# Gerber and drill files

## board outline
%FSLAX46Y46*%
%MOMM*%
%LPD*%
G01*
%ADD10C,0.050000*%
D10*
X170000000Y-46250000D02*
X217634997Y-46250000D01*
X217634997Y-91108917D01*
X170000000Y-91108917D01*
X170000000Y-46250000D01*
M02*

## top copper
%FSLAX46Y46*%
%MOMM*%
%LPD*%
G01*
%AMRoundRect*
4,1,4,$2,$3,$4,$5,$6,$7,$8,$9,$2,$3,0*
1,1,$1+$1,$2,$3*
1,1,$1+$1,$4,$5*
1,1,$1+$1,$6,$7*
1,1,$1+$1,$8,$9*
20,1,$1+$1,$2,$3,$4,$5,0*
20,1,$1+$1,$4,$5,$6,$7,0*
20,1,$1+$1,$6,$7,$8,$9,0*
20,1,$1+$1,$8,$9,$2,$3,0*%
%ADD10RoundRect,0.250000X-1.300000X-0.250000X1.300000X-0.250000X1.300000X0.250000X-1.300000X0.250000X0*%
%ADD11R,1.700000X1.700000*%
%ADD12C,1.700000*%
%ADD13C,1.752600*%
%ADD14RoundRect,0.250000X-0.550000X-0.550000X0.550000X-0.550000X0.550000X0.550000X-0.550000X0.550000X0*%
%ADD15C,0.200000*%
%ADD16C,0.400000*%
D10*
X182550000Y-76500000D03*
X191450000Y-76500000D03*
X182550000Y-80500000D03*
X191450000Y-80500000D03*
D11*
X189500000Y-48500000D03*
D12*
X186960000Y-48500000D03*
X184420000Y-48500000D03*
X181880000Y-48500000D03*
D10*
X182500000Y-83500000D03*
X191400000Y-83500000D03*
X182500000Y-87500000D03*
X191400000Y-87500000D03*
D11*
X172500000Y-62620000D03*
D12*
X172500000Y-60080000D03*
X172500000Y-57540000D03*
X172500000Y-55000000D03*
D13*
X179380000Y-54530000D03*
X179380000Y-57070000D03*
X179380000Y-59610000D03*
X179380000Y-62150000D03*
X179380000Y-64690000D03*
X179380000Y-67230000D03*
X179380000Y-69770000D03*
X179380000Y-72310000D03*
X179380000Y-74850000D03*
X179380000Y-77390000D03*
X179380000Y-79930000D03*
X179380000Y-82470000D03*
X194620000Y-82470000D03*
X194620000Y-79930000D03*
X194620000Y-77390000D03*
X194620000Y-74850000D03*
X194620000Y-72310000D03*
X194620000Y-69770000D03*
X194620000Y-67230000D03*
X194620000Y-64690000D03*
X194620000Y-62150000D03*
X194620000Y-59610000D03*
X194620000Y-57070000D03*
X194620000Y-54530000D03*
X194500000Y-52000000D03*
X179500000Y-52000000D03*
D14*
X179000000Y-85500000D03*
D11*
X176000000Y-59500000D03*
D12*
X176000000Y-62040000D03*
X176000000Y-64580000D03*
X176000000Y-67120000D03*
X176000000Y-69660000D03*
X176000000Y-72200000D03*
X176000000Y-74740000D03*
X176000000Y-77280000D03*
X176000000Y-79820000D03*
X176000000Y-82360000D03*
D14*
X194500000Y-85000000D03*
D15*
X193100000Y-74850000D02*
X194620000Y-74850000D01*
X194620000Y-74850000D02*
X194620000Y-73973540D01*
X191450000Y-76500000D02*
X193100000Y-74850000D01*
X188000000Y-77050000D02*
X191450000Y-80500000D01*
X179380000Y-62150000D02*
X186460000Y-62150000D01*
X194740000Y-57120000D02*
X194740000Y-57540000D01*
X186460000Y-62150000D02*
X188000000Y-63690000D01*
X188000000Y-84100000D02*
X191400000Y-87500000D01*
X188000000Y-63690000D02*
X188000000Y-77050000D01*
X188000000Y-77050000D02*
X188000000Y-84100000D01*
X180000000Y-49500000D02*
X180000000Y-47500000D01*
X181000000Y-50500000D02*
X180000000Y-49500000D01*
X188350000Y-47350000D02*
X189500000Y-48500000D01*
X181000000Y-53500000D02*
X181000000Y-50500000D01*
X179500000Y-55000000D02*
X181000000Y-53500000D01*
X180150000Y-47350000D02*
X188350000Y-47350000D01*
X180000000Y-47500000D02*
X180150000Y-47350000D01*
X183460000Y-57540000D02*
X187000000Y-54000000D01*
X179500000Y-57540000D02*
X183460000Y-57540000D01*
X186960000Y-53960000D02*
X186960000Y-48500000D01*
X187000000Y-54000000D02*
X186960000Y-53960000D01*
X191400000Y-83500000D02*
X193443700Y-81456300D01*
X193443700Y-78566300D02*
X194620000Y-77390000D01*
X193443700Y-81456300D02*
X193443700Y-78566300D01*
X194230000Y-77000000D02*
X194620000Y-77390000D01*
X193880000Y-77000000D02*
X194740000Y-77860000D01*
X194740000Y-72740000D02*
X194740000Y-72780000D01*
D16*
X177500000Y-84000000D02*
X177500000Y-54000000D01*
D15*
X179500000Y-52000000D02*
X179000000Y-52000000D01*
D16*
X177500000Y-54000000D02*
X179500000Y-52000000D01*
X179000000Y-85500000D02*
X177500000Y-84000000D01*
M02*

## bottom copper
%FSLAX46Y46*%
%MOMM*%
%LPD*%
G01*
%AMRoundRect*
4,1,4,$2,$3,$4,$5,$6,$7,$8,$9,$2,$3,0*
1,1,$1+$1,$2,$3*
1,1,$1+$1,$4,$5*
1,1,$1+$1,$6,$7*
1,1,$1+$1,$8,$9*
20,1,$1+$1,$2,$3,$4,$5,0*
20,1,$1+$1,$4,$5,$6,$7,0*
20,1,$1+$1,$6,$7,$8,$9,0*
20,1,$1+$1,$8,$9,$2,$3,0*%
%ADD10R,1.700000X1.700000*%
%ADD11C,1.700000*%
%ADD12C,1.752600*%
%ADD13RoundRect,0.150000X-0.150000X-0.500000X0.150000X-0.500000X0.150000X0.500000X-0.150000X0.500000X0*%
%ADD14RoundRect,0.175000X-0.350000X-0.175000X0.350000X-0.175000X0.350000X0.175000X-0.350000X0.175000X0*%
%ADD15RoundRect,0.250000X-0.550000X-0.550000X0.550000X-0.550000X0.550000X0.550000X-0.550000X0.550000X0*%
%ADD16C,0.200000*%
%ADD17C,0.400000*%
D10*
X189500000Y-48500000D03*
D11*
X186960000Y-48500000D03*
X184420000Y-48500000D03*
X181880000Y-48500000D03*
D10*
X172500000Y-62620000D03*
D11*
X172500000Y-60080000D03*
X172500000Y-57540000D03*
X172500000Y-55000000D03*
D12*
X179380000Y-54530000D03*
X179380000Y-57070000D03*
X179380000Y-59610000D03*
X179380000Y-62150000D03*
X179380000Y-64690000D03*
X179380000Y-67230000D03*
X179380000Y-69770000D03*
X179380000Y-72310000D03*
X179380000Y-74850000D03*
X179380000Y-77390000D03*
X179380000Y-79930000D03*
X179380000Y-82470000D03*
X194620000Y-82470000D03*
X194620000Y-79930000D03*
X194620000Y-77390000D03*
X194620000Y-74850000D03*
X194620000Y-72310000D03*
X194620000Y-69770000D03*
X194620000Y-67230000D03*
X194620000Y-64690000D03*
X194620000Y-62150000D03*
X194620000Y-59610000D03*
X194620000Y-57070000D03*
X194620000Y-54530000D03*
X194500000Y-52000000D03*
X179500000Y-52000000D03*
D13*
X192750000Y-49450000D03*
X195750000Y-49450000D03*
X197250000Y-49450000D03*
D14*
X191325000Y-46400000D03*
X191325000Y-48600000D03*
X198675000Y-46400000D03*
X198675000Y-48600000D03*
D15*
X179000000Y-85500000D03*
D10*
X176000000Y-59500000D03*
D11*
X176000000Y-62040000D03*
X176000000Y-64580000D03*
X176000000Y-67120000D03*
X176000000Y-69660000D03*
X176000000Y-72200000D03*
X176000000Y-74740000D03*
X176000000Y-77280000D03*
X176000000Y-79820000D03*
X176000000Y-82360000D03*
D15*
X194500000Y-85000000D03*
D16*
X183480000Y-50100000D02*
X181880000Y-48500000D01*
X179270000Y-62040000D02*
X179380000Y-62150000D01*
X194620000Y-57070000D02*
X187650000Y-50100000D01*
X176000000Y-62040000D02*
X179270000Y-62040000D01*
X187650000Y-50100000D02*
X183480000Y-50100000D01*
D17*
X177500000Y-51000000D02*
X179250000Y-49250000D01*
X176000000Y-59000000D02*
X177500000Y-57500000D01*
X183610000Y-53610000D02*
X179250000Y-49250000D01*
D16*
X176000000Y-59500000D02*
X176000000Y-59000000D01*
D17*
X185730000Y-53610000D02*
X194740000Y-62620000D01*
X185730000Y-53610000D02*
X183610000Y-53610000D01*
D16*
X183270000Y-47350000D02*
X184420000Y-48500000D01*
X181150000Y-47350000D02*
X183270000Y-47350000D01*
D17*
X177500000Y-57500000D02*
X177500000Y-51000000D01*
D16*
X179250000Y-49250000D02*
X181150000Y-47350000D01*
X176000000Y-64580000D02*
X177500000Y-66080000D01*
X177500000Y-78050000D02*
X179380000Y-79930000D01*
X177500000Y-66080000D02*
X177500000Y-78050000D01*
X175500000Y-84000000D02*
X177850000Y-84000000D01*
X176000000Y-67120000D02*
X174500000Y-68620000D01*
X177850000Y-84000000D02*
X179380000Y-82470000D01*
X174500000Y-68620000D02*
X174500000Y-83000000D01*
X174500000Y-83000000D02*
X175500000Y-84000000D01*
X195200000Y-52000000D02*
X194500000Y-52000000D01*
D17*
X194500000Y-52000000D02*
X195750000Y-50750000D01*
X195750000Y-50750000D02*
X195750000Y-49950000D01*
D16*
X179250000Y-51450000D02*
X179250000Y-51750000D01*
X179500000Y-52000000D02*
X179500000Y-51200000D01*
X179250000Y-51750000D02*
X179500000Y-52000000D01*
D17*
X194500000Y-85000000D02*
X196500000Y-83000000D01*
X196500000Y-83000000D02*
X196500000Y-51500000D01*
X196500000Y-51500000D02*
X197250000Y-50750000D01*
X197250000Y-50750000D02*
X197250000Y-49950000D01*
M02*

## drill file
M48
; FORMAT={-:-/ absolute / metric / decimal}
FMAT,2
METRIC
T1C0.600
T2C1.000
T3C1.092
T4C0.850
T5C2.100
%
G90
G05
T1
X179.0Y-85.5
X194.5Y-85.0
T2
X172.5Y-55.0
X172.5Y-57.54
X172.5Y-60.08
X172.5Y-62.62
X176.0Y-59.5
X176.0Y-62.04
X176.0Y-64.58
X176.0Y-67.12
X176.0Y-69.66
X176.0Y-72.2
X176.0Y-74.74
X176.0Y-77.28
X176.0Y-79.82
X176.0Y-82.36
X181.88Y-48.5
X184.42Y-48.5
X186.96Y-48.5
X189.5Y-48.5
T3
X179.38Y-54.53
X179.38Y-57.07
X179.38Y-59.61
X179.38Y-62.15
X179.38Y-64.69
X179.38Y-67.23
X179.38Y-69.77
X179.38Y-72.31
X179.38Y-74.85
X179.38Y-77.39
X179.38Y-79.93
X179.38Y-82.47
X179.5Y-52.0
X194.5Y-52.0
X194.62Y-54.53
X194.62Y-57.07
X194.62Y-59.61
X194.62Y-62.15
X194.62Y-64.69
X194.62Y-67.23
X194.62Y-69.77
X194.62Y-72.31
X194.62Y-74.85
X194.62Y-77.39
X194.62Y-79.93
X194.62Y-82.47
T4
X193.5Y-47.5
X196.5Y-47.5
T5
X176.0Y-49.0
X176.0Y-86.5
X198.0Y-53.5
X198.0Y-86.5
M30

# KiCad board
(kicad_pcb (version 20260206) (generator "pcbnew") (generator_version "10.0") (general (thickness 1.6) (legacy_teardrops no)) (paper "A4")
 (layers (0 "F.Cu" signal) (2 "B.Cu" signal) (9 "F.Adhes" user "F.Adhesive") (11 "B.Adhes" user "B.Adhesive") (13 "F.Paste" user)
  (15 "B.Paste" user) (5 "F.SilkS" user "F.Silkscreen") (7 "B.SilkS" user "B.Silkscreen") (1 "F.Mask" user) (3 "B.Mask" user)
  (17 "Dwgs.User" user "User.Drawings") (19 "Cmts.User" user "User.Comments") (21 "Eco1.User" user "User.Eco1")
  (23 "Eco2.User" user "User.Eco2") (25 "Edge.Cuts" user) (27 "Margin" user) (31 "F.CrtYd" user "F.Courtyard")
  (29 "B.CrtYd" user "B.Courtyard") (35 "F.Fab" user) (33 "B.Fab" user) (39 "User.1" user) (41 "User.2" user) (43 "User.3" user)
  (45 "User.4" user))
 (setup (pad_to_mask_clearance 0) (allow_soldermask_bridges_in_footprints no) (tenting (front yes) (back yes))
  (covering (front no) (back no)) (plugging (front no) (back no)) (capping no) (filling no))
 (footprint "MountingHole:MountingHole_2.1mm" (layer "F.Cu") (at 176 49)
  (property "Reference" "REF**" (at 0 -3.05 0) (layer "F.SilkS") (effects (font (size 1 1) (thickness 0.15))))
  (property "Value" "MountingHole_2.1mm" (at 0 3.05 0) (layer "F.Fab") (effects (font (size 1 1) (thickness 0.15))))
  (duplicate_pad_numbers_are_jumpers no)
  (pad "" np_thru_hole circle (at 0 0) (size 2.1 2.1) (drill 2.1) (layers "*.Cu" "*.Mask")))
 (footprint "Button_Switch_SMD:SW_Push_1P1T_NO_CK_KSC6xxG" (layer "F.Cu") (at 187 78.5)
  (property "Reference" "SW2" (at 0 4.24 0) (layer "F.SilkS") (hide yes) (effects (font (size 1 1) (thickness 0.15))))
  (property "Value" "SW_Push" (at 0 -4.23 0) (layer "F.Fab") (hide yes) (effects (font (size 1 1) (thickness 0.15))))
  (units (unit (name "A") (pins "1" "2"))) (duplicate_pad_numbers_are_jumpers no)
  (pad "1" smd roundrect (at -4.45 -2) (size 3.1 1) (layers "F.Cu" "F.Mask" "F.Paste") (roundrect_rratio 0.25) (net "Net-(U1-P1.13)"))
  (pad "1" smd roundrect (at 4.45 -2) (size 3.1 1) (layers "F.Cu" "F.Mask" "F.Paste") (roundrect_rratio 0.25) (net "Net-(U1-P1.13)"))
  (pad "2" smd roundrect (at -4.45 2) (size 3.1 1) (layers "F.Cu" "F.Mask" "F.Paste") (roundrect_rratio 0.25) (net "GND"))
  (pad "2" smd roundrect (at 4.45 2) (size 3.1 1) (layers "F.Cu" "F.Mask" "F.Paste") (roundrect_rratio 0.25) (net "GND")))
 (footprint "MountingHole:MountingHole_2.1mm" (layer "F.Cu") (at 198 86.5)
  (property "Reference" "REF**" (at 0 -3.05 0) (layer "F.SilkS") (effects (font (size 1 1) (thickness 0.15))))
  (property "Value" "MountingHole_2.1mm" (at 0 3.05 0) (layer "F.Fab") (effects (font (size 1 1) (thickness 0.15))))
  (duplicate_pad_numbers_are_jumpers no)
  (pad "" np_thru_hole circle (at 0 0) (size 2.1 2.1) (drill 2.1) (layers "*.Cu" "*.Mask")))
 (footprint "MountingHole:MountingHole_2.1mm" (layer "F.Cu") (at 176 86.5)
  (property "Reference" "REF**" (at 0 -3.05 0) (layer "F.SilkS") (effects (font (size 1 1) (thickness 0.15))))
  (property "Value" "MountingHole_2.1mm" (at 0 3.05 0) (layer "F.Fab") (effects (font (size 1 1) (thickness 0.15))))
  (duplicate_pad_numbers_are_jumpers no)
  (pad "" np_thru_hole circle (at 0 0) (size 2.1 2.1) (drill 2.1) (layers "*.Cu" "*.Mask")))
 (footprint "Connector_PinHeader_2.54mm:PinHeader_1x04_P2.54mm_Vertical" (layer "F.Cu") (at 189.5 48.5 -90)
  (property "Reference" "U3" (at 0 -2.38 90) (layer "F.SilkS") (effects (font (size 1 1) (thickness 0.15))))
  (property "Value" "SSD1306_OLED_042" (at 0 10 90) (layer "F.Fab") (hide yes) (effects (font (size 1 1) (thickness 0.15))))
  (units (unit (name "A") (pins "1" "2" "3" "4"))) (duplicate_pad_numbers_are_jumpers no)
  (pad "1" thru_hole rect (at 0 0 270) (size 1.7 1.7) (drill 1) (layers "*.Cu" "*.Mask") (remove_unused_layers no)
   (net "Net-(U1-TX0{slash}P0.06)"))
  (pad "2" thru_hole circle (at 0 2.54 270) (size 1.7 1.7) (drill 1) (layers "*.Cu" "*.Mask") (remove_unused_layers no)
   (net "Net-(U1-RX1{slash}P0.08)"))
  (pad "3" thru_hole circle (at 0 5.08 270) (size 1.7 1.7) (drill 1) (layers "*.Cu" "*.Mask") (remove_unused_layers no) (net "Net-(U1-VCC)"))
  (pad "4" thru_hole circle (at 0 7.62 270) (size 1.7 1.7) (drill 1) (layers "*.Cu" "*.Mask") (remove_unused_layers no) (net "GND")))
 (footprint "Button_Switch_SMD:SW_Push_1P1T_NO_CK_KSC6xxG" (layer "F.Cu") (at 186.95 85.5)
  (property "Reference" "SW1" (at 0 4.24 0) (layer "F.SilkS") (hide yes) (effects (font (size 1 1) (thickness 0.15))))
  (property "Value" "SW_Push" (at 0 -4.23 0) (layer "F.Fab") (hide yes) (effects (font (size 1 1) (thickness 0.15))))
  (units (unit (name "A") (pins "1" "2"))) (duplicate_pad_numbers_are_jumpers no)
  (pad "1" smd roundrect (at -4.45 -2) (size 3.1 1) (layers "F.Cu" "F.Mask" "F.Paste") (roundrect_rratio 0.25) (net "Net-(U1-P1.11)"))
  (pad "1" smd roundrect (at 4.45 -2) (size 3.1 1) (layers "F.Cu" "F.Mask" "F.Paste") (roundrect_rratio 0.25) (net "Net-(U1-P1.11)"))
  (pad "2" smd roundrect (at -4.45 2) (size 3.1 1) (layers "F.Cu" "F.Mask" "F.Paste") (roundrect_rratio 0.25) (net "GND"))
  (pad "2" smd roundrect (at 4.45 2) (size 3.1 1) (layers "F.Cu" "F.Mask" "F.Paste") (roundrect_rratio 0.25) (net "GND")))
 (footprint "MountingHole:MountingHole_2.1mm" (layer "F.Cu") (at 198 53.5)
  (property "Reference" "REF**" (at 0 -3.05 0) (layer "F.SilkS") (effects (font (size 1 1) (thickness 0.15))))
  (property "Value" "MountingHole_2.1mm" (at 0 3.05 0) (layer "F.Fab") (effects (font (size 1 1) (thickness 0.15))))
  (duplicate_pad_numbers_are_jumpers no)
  (pad "" np_thru_hole circle (at 0 0) (size 2.1 2.1) (drill 2.1) (layers "*.Cu" "*.Mask")))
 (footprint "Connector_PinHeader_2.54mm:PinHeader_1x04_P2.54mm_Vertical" (layer "F.Cu") (at 172.5 62.62 180)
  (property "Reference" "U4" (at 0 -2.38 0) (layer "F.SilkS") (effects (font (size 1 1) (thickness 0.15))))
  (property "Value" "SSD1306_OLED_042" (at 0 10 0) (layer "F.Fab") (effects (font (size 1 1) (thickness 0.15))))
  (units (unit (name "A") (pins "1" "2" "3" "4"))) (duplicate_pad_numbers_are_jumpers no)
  (pad "1" thru_hole rect (at 0 0 180) (size 1.7 1.7) (drill 1) (layers "*.Cu" "*.Mask") (remove_unused_layers no)
   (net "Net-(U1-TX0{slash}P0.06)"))
  (pad "2" thru_hole circle (at 0 2.54 180) (size 1.7 1.7) (drill 1) (layers "*.Cu" "*.Mask") (remove_unused_layers no)
   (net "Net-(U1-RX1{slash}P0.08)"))
  (pad "3" thru_hole circle (at 0 5.08 180) (size 1.7 1.7) (drill 1) (layers "*.Cu" "*.Mask") (remove_unused_layers no) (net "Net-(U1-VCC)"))
  (pad "4" thru_hole circle (at 0 7.62 180) (size 1.7 1.7) (drill 1) (layers "*.Cu" "*.Mask") (remove_unused_layers no) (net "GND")))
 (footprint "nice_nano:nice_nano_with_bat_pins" (layer "F.Cu") (at 187 68.5 -90)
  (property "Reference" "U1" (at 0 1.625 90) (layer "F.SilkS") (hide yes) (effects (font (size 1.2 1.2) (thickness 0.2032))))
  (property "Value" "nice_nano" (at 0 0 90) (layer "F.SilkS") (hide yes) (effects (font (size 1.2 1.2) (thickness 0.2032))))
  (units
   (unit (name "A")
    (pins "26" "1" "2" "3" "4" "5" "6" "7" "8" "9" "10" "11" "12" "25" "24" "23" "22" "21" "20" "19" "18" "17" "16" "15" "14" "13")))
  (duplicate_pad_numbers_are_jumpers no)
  (pad "1" thru_hole circle (at -13.97 7.62 270) (size 1.7526 1.7526) (drill 1.0922) (layers "*.Cu" "*.SilkS" "*.Mask")
   (remove_unused_layers no) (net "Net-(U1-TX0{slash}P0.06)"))
  (pad "2" thru_hole circle (at -11.43 7.62 270) (size 1.7526 1.7526) (drill 1.0922) (layers "*.Cu" "*.SilkS" "*.Mask")
   (remove_unused_layers no) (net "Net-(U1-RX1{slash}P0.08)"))
  (pad "3" thru_hole circle (at -8.89 7.62 270) (size 1.7526 1.7526) (drill 1.0922) (layers "*.Cu" "*.SilkS" "*.Mask")
   (remove_unused_layers no) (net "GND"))
  (pad "4" thru_hole circle (at -6.35 7.62 270) (size 1.7526 1.7526) (drill 1.0922) (layers "*.Cu" "*.SilkS" "*.Mask")
   (remove_unused_layers no) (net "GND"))
  (pad "5" thru_hole circle (at -3.81 7.62 270) (size 1.7526 1.7526) (drill 1.0922) (layers "*.Cu" "*.SilkS" "*.Mask")
   (remove_unused_layers no) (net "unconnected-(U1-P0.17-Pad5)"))
  (pad "6" thru_hole circle (at -1.27 7.62 270) (size 1.7526 1.7526) (drill 1.0922) (layers "*.Cu" "*.SilkS" "*.Mask")
   (remove_unused_layers no) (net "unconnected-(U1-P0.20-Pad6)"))
  (pad "7" thru_hole circle (at 1.27 7.62 270) (size 1.7526 1.7526) (drill 1.0922) (layers "*.Cu" "*.SilkS" "*.Mask")
   (remove_unused_layers no) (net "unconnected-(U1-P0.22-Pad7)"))
  (pad "8" thru_hole circle (at 3.81 7.62 270) (size 1.7526 1.7526) (drill 1.0922) (layers "*.Cu" "*.SilkS" "*.Mask")
   (remove_unused_layers no) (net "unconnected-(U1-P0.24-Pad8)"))
  (pad "9" thru_hole circle (at 6.35 7.62 270) (size 1.7526 1.7526) (drill 1.0922) (layers "*.Cu" "*.SilkS" "*.Mask")
   (remove_unused_layers no) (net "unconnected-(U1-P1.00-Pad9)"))
  (pad "10" thru_hole circle (at 8.89 7.62 270) (size 1.7526 1.7526) (drill 1.0922) (layers "*.Cu" "*.SilkS" "*.Mask")
   (remove_unused_layers no) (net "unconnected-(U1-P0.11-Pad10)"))
  (pad "11" thru_hole circle (at 11.43 7.62 270) (size 1.7526 1.7526) (drill 1.0922) (layers "*.Cu" "*.SilkS" "*.Mask")
   (remove_unused_layers no) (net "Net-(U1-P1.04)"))
  (pad "12" thru_hole circle (at 13.97 7.62 270) (size 1.7526 1.7526) (drill 1.0922) (layers "*.Cu" "*.SilkS" "*.Mask")
   (remove_unused_layers no) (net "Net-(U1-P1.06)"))
  (pad "13" thru_hole circle (at 13.97 -7.62 270) (size 1.7526 1.7526) (drill 1.0922) (layers "*.Cu" "*.SilkS" "*.Mask")
   (remove_unused_layers no) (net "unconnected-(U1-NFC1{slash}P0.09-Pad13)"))
  (pad "14" thru_hole circle (at 11.43 -7.62 270) (size 1.7526 1.7526) (drill 1.0922) (layers "*.Cu" "*.SilkS" "*.Mask")
   (remove_unused_layers no) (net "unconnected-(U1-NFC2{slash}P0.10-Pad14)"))
  (pad "15" thru_hole circle (at 8.89 -7.62 270) (size 1.7526 1.7526) (drill 1.0922) (layers "*.Cu" "*.SilkS" "*.Mask")
   (remove_unused_layers no) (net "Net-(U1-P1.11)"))
  (pad "16" thru_hole circle (at 6.35 -7.62 270) (size 1.7526 1.7526) (drill 1.0922) (layers "*.Cu" "*.SilkS" "*.Mask")
   (remove_unused_layers no) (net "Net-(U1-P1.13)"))
  (pad "17" thru_hole circle (at 3.81 -7.62 270) (size 1.7526 1.7526) (drill 1.0922) (layers "*.Cu" "*.SilkS" "*.Mask")
   (remove_unused_layers no) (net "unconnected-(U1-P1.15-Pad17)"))
  (pad "18" thru_hole circle (at 1.27 -7.62 270) (size 1.7526 1.7526) (drill 1.0922) (layers "*.Cu" "*.SilkS" "*.Mask")
   (remove_unused_layers no) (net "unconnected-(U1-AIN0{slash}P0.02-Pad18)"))
  (pad "19" thru_hole circle (at -1.27 -7.62 270) (size 1.7526 1.7526) (drill 1.0922) (layers "*.Cu" "*.SilkS" "*.Mask")
   (remove_unused_layers no) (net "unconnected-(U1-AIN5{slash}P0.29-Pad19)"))
  (pad "20" thru_hole circle (at -3.81 -7.62 270) (size 1.7526 1.7526) (drill 1.0922) (layers "*.Cu" "*.SilkS" "*.Mask")
   (remove_unused_layers no) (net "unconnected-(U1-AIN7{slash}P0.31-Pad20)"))
  (pad "21" thru_hole circle (at -6.35 -7.62 270) (size 1.7526 1.7526) (drill 1.0922) (layers "*.Cu" "*.SilkS" "*.Mask")
   (remove_unused_layers no) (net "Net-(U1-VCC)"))
  (pad "22" thru_hole circle (at -8.89 -7.62 270) (size 1.7526 1.7526) (drill 1.0922) (layers "*.Cu" "*.SilkS" "*.Mask")
   (remove_unused_layers no) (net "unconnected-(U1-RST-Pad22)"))
  (pad "23" thru_hole circle (at -11.43 -7.62 270) (size 1.7526 1.7526) (drill 1.0922) (layers "*.Cu" "*.SilkS" "*.Mask")
   (remove_unused_layers no) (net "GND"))
  (pad "24" thru_hole circle (at -13.97 -7.62 270) (size 1.7526 1.7526) (drill 1.0922) (layers "*.Cu" "*.SilkS" "*.Mask")
   (remove_unused_layers no) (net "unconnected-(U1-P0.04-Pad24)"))
  (pad "25" thru_hole circle (at -16.5 -7.5 270) (size 1.7526 1.7526) (drill 1.0922) (layers "*.Cu" "*.SilkS" "*.Mask")
   (remove_unused_layers no) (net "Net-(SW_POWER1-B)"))
  (pad "26" thru_hole circle (at -16.5 7.5 270) (size 1.7526 1.7526) (drill 1.0922) (layers "*.Cu" "*.SilkS" "*.Mask")
   (remove_unused_layers no) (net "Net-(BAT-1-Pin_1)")))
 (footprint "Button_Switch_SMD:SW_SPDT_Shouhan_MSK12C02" (layer "B.Cu") (at 195 47.5)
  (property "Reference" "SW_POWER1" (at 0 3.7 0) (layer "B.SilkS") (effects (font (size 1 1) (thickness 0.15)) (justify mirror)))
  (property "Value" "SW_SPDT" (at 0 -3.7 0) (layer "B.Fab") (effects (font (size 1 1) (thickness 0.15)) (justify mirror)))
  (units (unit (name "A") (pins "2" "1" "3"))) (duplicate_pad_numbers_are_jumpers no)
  (pad "" np_thru_hole circle (at -1.5 0) (size 0.85 0.85) (drill 0.85) (layers "*.Mask"))
  (pad "" np_thru_hole circle (at 1.5 0) (size 0.85 0.85) (drill 0.85) (layers "*.Mask"))
  (pad "1" smd roundrect (at -2.25 1.95) (size 0.6 1.3) (layers "B.Cu" "B.Mask" "B.Paste") (roundrect_rratio 0.25)
   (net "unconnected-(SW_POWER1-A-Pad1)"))
  (pad "2" smd roundrect (at 0.75 1.95) (size 0.6 1.3) (layers "B.Cu" "B.Mask" "B.Paste") (roundrect_rratio 0.25) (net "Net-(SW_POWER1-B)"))
  (pad "3" smd roundrect (at 2.25 1.95) (size 0.6 1.3) (layers "B.Cu" "B.Mask" "B.Paste") (roundrect_rratio 0.25) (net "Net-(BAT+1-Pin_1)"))
  (pad "SH" smd roundrect (at -3.675 -1.1) (size 1.05 0.7) (layers "B.Cu" "B.Mask" "B.Paste") (roundrect_rratio 0.25))
  (pad "SH" smd roundrect (at -3.675 1.1) (size 1.05 0.7) (layers "B.Cu" "B.Mask" "B.Paste") (roundrect_rratio 0.25))
  (pad "SH" smd roundrect (at 3.675 -1.1) (size 1.05 0.7) (layers "B.Cu" "B.Mask" "B.Paste") (roundrect_rratio 0.25))
  (pad "SH" smd roundrect (at 3.675 1.1) (size 1.05 0.7) (layers "B.Cu" "B.Mask" "B.Paste") (roundrect_rratio 0.25)))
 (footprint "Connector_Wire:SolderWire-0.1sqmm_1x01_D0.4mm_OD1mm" (layer "B.Cu") (at 179 85.5)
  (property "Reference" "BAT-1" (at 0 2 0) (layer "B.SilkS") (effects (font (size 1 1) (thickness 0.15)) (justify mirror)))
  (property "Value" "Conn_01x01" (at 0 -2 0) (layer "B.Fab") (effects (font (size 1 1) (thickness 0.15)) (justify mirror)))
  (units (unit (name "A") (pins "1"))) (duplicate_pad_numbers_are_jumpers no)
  (pad "1" thru_hole roundrect (at 0 0) (size 1.6 1.6) (drill 0.6) (layers "*.Cu" "*.Mask") (remove_unused_layers no)
   (roundrect_rratio 0.15625) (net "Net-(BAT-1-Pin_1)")))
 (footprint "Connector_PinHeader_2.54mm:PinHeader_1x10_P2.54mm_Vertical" (layer "B.Cu") (at 176 59.5 180)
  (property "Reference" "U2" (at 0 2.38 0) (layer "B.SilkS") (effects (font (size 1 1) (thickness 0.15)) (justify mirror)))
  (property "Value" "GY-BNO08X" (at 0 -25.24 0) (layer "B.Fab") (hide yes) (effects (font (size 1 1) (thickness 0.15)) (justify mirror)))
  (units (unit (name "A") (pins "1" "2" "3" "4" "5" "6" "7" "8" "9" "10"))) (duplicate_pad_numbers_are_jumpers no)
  (pad "1" thru_hole rect (at 0 0 180) (size 1.7 1.7) (drill 1) (layers "*.Cu" "*.Mask") (remove_unused_layers no) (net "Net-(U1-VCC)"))
  (pad "2" thru_hole circle (at 0 -2.54 180) (size 1.7 1.7) (drill 1) (layers "*.Cu" "*.Mask") (remove_unused_layers no) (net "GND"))
  (pad "3" thru_hole circle (at 0 -5.08 180) (size 1.7 1.7) (drill 1) (layers "*.Cu" "*.Mask") (remove_unused_layers no)
   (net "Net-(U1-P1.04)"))
  (pad "4" thru_hole circle (at 0 -7.62 180) (size 1.7 1.7) (drill 1) (layers "*.Cu" "*.Mask") (remove_unused_layers no)
   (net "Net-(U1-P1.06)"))
  (pad "5" thru_hole circle (at 0 -10.16 180) (size 1.7 1.7) (drill 1) (layers "*.Cu" "*.Mask") (remove_unused_layers no)
   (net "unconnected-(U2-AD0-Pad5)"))
  (pad "6" thru_hole circle (at 0 -12.7 180) (size 1.7 1.7) (drill 1) (layers "*.Cu" "*.Mask") (remove_unused_layers no)
   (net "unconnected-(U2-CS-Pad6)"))
  (pad "7" thru_hole circle (at 0 -15.24 180) (size 1.7 1.7) (drill 1) (layers "*.Cu" "*.Mask") (remove_unused_layers no)
   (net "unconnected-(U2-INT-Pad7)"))
  (pad "8" thru_hole circle (at 0 -17.78 180) (size 1.7 1.7) (drill 1) (layers "*.Cu" "*.Mask") (remove_unused_layers no)
   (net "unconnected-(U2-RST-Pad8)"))
  (pad "9" thru_hole circle (at 0 -20.32 180) (size 1.7 1.7) (drill 1) (layers "*.Cu" "*.Mask") (remove_unused_layers no)
   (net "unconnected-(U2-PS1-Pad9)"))
  (pad "10" thru_hole circle (at 0 -22.86 180) (size 1.7 1.7) (drill 1) (layers "*.Cu" "*.Mask") (remove_unused_layers no)
   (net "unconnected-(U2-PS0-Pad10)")))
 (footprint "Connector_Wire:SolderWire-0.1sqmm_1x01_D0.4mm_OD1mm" (layer "B.Cu") (at 194.5 85)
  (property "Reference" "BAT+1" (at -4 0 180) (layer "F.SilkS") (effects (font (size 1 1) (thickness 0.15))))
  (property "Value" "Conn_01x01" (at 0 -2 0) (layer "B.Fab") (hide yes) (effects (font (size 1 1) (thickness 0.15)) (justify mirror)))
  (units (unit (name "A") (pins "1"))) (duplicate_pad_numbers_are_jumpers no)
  (pad "1" thru_hole roundrect (at 0 0) (size 1.6 1.6) (drill 0.6) (layers "*.Cu" "*.Mask") (remove_unused_layers no)
   (roundrect_rratio 0.15625) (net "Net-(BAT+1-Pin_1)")))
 (gr_rect (start 170 46.25) (end 217.634997 91.108917) (stroke (width 0.05) (type default)) (fill no) (layer "Edge.Cuts"))
 (segment (start 193.1 74.85) (end 194.62 74.85) (width 0.2) (layer "F.Cu") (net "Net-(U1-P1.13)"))
 (segment (start 194.62 74.85) (end 194.62 73.97354) (width 0.2) (layer "F.Cu") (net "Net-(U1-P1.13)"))
 (segment (start 191.45 76.5) (end 193.1 74.85) (width 0.2) (layer "F.Cu") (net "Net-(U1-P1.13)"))
 (segment (start 188 77.05) (end 191.45 80.5) (width 0.2) (layer "F.Cu") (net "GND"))
 (segment (start 179.38 62.15) (end 186.46 62.15) (width 0.2) (layer "F.Cu") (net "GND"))
 (segment (start 194.74 57.12) (end 194.74 57.54) (width 0.2) (layer "F.Cu") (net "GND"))
 (segment (start 186.46 62.15) (end 188 63.69) (width 0.2) (layer "F.Cu") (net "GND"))
 (segment (start 188 84.1) (end 191.4 87.5) (width 0.2) (layer "F.Cu") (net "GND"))
 (segment (start 188 63.69) (end 188 77.05) (width 0.2) (layer "F.Cu") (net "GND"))
 (segment (start 188 77.05) (end 188 84.1) (width 0.2) (layer "F.Cu") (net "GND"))
 (segment (start 183.48 50.1) (end 181.88 48.5) (width 0.2) (layer "B.Cu") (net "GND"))
 (segment (start 179.27 62.04) (end 179.38 62.15) (width 0.2) (layer "B.Cu") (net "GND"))
 (segment (start 194.62 57.07) (end 187.65 50.1) (width 0.2) (layer "B.Cu") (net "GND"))
 (segment (start 176 62.04) (end 179.27 62.04) (width 0.2) (layer "B.Cu") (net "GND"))
 (segment (start 187.65 50.1) (end 183.48 50.1) (width 0.2) (layer "B.Cu") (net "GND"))
 (segment (start 180 49.5) (end 180 47.5) (width 0.2) (layer "F.Cu") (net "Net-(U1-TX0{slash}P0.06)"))
 (segment (start 181 50.5) (end 180 49.5) (width 0.2) (layer "F.Cu") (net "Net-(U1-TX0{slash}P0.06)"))
 (segment (start 188.35 47.35) (end 189.5 48.5) (width 0.2) (layer "F.Cu") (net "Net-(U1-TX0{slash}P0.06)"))
 (segment (start 181 53.5) (end 181 50.5) (width 0.2) (layer "F.Cu") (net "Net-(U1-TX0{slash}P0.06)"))
 (segment (start 179.5 55) (end 181 53.5) (width 0.2) (layer "F.Cu") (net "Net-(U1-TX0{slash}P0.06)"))
 (segment (start 180.15 47.35) (end 188.35 47.35) (width 0.2) (layer "F.Cu") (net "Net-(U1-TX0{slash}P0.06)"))
 (segment (start 180 47.5) (end 180.15 47.35) (width 0.2) (layer "F.Cu") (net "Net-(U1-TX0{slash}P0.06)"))
 (segment (start 183.46 57.54) (end 187 54) (width 0.2) (layer "F.Cu") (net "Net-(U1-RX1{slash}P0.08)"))
 (segment (start 179.5 57.54) (end 183.46 57.54) (width 0.2) (layer "F.Cu") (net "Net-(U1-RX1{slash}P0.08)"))
 (segment (start 186.96 53.96) (end 186.96 48.5) (width 0.2) (layer "F.Cu") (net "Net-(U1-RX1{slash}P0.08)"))
 (segment (start 187 54) (end 186.96 53.96) (width 0.2) (layer "F.Cu") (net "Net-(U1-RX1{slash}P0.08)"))
 (segment (start 177.5 51) (end 179.25 49.25) (width 0.4) (layer "B.Cu") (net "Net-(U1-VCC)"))
 (segment (start 176 59) (end 177.5 57.5) (width 0.4) (layer "B.Cu") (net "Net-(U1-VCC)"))
 (segment (start 183.61 53.61) (end 179.25 49.25) (width 0.4) (layer "B.Cu") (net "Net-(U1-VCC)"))
 (segment (start 176 59.5) (end 176 59) (width 0.2) (layer "B.Cu") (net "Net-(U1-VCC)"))
 (segment (start 185.73 53.61) (end 194.74 62.62) (width 0.4) (layer "B.Cu") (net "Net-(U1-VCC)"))
 (segment (start 185.73 53.61) (end 183.61 53.61) (width 0.4) (layer "B.Cu") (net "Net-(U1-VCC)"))
 (segment (start 183.27 47.35) (end 184.42 48.5) (width 0.2) (layer "B.Cu") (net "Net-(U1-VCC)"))
 (segment (start 181.15 47.35) (end 183.27 47.35) (width 0.2) (layer "B.Cu") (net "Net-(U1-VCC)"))
 (segment (start 177.5 57.5) (end 177.5 51) (width 0.4) (layer "B.Cu") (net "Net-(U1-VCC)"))
 (segment (start 179.25 49.25) (end 181.15 47.35) (width 0.2) (layer "B.Cu") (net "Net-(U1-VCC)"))
 (segment (start 191.4 83.5) (end 193.4437 81.4563) (width 0.2) (layer "F.Cu") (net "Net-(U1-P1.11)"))
 (segment (start 193.4437 78.5663) (end 194.62 77.39) (width 0.2) (layer "F.Cu") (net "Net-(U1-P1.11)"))
 (segment (start 193.4437 81.4563) (end 193.4437 78.5663) (width 0.2) (layer "F.Cu") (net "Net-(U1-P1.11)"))
 (segment (start 194.23 77) (end 194.62 77.39) (width 0.2) (layer "F.Cu") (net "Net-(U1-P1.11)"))
 (segment (start 193.88 77) (end 194.74 77.86) (width 0.2) (layer "F.Cu") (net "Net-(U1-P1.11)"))
 (segment (start 176 64.58) (end 177.5 66.08) (width 0.2) (layer "B.Cu") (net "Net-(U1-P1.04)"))
 (segment (start 177.5 78.05) (end 179.38 79.93) (width 0.2) (layer "B.Cu") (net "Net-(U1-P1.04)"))
 (segment (start 177.5 66.08) (end 177.5 78.05) (width 0.2) (layer "B.Cu") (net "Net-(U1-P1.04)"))
 (segment (start 175.5 84) (end 177.85 84) (width 0.2) (layer "B.Cu") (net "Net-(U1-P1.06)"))
 (segment (start 176 67.12) (end 174.5 68.62) (width 0.2) (layer "B.Cu") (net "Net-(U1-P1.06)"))
 (segment (start 177.85 84) (end 179.38 82.47) (width 0.2) (layer "B.Cu") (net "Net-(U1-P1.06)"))
 (segment (start 174.5 68.62) (end 174.5 83) (width 0.2) (layer "B.Cu") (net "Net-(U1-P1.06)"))
 (segment (start 174.5 83) (end 175.5 84) (width 0.2) (layer "B.Cu") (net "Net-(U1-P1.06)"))
 (segment (start 194.74 72.74) (end 194.74 72.78) (width 0.2) (layer "F.Cu") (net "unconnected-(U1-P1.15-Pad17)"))
 (segment (start 195.2 52) (end 194.5 52) (width 0.2) (layer "B.Cu") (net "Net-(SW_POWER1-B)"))
 (segment (start 194.5 52) (end 195.75 50.75) (width 0.4) (layer "B.Cu") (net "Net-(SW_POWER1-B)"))
 (segment (start 195.75 50.75) (end 195.75 49.95) (width 0.4) (layer "B.Cu") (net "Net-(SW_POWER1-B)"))
 (segment (start 177.5 84) (end 177.5 54) (width 0.4) (layer "F.Cu") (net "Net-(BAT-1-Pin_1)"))
 (segment (start 179.5 52) (end 179 52) (width 0.2) (layer "F.Cu") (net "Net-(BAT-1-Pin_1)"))
 (segment (start 177.5 54) (end 179.5 52) (width 0.4) (layer "F.Cu") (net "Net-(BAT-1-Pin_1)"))
 (segment (start 179 85.5) (end 177.5 84) (width 0.4) (layer "F.Cu") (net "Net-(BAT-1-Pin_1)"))
 (segment (start 179.25 51.45) (end 179.25 51.75) (width 0.2) (layer "B.Cu") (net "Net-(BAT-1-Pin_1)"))
 (segment (start 179.5 52) (end 179.5 51.2) (width 0.2) (layer "B.Cu") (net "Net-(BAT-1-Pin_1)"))
 (segment (start 179.25 51.75) (end 179.5 52) (width 0.2) (layer "B.Cu") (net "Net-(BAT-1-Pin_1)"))
 (segment (start 194.5 85) (end 196.5 83) (width 0.4) (layer "B.Cu") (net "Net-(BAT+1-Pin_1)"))
 (segment (start 196.5 83) (end 196.5 51.5) (width 0.4) (layer "B.Cu") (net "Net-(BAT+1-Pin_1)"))
 (segment (start 196.5 51.5) (end 197.25 50.75) (width 0.4) (layer "B.Cu") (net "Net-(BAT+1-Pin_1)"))
 (segment (start 197.25 50.75) (end 197.25 49.95) (width 0.4) (layer "B.Cu") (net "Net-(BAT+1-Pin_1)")))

